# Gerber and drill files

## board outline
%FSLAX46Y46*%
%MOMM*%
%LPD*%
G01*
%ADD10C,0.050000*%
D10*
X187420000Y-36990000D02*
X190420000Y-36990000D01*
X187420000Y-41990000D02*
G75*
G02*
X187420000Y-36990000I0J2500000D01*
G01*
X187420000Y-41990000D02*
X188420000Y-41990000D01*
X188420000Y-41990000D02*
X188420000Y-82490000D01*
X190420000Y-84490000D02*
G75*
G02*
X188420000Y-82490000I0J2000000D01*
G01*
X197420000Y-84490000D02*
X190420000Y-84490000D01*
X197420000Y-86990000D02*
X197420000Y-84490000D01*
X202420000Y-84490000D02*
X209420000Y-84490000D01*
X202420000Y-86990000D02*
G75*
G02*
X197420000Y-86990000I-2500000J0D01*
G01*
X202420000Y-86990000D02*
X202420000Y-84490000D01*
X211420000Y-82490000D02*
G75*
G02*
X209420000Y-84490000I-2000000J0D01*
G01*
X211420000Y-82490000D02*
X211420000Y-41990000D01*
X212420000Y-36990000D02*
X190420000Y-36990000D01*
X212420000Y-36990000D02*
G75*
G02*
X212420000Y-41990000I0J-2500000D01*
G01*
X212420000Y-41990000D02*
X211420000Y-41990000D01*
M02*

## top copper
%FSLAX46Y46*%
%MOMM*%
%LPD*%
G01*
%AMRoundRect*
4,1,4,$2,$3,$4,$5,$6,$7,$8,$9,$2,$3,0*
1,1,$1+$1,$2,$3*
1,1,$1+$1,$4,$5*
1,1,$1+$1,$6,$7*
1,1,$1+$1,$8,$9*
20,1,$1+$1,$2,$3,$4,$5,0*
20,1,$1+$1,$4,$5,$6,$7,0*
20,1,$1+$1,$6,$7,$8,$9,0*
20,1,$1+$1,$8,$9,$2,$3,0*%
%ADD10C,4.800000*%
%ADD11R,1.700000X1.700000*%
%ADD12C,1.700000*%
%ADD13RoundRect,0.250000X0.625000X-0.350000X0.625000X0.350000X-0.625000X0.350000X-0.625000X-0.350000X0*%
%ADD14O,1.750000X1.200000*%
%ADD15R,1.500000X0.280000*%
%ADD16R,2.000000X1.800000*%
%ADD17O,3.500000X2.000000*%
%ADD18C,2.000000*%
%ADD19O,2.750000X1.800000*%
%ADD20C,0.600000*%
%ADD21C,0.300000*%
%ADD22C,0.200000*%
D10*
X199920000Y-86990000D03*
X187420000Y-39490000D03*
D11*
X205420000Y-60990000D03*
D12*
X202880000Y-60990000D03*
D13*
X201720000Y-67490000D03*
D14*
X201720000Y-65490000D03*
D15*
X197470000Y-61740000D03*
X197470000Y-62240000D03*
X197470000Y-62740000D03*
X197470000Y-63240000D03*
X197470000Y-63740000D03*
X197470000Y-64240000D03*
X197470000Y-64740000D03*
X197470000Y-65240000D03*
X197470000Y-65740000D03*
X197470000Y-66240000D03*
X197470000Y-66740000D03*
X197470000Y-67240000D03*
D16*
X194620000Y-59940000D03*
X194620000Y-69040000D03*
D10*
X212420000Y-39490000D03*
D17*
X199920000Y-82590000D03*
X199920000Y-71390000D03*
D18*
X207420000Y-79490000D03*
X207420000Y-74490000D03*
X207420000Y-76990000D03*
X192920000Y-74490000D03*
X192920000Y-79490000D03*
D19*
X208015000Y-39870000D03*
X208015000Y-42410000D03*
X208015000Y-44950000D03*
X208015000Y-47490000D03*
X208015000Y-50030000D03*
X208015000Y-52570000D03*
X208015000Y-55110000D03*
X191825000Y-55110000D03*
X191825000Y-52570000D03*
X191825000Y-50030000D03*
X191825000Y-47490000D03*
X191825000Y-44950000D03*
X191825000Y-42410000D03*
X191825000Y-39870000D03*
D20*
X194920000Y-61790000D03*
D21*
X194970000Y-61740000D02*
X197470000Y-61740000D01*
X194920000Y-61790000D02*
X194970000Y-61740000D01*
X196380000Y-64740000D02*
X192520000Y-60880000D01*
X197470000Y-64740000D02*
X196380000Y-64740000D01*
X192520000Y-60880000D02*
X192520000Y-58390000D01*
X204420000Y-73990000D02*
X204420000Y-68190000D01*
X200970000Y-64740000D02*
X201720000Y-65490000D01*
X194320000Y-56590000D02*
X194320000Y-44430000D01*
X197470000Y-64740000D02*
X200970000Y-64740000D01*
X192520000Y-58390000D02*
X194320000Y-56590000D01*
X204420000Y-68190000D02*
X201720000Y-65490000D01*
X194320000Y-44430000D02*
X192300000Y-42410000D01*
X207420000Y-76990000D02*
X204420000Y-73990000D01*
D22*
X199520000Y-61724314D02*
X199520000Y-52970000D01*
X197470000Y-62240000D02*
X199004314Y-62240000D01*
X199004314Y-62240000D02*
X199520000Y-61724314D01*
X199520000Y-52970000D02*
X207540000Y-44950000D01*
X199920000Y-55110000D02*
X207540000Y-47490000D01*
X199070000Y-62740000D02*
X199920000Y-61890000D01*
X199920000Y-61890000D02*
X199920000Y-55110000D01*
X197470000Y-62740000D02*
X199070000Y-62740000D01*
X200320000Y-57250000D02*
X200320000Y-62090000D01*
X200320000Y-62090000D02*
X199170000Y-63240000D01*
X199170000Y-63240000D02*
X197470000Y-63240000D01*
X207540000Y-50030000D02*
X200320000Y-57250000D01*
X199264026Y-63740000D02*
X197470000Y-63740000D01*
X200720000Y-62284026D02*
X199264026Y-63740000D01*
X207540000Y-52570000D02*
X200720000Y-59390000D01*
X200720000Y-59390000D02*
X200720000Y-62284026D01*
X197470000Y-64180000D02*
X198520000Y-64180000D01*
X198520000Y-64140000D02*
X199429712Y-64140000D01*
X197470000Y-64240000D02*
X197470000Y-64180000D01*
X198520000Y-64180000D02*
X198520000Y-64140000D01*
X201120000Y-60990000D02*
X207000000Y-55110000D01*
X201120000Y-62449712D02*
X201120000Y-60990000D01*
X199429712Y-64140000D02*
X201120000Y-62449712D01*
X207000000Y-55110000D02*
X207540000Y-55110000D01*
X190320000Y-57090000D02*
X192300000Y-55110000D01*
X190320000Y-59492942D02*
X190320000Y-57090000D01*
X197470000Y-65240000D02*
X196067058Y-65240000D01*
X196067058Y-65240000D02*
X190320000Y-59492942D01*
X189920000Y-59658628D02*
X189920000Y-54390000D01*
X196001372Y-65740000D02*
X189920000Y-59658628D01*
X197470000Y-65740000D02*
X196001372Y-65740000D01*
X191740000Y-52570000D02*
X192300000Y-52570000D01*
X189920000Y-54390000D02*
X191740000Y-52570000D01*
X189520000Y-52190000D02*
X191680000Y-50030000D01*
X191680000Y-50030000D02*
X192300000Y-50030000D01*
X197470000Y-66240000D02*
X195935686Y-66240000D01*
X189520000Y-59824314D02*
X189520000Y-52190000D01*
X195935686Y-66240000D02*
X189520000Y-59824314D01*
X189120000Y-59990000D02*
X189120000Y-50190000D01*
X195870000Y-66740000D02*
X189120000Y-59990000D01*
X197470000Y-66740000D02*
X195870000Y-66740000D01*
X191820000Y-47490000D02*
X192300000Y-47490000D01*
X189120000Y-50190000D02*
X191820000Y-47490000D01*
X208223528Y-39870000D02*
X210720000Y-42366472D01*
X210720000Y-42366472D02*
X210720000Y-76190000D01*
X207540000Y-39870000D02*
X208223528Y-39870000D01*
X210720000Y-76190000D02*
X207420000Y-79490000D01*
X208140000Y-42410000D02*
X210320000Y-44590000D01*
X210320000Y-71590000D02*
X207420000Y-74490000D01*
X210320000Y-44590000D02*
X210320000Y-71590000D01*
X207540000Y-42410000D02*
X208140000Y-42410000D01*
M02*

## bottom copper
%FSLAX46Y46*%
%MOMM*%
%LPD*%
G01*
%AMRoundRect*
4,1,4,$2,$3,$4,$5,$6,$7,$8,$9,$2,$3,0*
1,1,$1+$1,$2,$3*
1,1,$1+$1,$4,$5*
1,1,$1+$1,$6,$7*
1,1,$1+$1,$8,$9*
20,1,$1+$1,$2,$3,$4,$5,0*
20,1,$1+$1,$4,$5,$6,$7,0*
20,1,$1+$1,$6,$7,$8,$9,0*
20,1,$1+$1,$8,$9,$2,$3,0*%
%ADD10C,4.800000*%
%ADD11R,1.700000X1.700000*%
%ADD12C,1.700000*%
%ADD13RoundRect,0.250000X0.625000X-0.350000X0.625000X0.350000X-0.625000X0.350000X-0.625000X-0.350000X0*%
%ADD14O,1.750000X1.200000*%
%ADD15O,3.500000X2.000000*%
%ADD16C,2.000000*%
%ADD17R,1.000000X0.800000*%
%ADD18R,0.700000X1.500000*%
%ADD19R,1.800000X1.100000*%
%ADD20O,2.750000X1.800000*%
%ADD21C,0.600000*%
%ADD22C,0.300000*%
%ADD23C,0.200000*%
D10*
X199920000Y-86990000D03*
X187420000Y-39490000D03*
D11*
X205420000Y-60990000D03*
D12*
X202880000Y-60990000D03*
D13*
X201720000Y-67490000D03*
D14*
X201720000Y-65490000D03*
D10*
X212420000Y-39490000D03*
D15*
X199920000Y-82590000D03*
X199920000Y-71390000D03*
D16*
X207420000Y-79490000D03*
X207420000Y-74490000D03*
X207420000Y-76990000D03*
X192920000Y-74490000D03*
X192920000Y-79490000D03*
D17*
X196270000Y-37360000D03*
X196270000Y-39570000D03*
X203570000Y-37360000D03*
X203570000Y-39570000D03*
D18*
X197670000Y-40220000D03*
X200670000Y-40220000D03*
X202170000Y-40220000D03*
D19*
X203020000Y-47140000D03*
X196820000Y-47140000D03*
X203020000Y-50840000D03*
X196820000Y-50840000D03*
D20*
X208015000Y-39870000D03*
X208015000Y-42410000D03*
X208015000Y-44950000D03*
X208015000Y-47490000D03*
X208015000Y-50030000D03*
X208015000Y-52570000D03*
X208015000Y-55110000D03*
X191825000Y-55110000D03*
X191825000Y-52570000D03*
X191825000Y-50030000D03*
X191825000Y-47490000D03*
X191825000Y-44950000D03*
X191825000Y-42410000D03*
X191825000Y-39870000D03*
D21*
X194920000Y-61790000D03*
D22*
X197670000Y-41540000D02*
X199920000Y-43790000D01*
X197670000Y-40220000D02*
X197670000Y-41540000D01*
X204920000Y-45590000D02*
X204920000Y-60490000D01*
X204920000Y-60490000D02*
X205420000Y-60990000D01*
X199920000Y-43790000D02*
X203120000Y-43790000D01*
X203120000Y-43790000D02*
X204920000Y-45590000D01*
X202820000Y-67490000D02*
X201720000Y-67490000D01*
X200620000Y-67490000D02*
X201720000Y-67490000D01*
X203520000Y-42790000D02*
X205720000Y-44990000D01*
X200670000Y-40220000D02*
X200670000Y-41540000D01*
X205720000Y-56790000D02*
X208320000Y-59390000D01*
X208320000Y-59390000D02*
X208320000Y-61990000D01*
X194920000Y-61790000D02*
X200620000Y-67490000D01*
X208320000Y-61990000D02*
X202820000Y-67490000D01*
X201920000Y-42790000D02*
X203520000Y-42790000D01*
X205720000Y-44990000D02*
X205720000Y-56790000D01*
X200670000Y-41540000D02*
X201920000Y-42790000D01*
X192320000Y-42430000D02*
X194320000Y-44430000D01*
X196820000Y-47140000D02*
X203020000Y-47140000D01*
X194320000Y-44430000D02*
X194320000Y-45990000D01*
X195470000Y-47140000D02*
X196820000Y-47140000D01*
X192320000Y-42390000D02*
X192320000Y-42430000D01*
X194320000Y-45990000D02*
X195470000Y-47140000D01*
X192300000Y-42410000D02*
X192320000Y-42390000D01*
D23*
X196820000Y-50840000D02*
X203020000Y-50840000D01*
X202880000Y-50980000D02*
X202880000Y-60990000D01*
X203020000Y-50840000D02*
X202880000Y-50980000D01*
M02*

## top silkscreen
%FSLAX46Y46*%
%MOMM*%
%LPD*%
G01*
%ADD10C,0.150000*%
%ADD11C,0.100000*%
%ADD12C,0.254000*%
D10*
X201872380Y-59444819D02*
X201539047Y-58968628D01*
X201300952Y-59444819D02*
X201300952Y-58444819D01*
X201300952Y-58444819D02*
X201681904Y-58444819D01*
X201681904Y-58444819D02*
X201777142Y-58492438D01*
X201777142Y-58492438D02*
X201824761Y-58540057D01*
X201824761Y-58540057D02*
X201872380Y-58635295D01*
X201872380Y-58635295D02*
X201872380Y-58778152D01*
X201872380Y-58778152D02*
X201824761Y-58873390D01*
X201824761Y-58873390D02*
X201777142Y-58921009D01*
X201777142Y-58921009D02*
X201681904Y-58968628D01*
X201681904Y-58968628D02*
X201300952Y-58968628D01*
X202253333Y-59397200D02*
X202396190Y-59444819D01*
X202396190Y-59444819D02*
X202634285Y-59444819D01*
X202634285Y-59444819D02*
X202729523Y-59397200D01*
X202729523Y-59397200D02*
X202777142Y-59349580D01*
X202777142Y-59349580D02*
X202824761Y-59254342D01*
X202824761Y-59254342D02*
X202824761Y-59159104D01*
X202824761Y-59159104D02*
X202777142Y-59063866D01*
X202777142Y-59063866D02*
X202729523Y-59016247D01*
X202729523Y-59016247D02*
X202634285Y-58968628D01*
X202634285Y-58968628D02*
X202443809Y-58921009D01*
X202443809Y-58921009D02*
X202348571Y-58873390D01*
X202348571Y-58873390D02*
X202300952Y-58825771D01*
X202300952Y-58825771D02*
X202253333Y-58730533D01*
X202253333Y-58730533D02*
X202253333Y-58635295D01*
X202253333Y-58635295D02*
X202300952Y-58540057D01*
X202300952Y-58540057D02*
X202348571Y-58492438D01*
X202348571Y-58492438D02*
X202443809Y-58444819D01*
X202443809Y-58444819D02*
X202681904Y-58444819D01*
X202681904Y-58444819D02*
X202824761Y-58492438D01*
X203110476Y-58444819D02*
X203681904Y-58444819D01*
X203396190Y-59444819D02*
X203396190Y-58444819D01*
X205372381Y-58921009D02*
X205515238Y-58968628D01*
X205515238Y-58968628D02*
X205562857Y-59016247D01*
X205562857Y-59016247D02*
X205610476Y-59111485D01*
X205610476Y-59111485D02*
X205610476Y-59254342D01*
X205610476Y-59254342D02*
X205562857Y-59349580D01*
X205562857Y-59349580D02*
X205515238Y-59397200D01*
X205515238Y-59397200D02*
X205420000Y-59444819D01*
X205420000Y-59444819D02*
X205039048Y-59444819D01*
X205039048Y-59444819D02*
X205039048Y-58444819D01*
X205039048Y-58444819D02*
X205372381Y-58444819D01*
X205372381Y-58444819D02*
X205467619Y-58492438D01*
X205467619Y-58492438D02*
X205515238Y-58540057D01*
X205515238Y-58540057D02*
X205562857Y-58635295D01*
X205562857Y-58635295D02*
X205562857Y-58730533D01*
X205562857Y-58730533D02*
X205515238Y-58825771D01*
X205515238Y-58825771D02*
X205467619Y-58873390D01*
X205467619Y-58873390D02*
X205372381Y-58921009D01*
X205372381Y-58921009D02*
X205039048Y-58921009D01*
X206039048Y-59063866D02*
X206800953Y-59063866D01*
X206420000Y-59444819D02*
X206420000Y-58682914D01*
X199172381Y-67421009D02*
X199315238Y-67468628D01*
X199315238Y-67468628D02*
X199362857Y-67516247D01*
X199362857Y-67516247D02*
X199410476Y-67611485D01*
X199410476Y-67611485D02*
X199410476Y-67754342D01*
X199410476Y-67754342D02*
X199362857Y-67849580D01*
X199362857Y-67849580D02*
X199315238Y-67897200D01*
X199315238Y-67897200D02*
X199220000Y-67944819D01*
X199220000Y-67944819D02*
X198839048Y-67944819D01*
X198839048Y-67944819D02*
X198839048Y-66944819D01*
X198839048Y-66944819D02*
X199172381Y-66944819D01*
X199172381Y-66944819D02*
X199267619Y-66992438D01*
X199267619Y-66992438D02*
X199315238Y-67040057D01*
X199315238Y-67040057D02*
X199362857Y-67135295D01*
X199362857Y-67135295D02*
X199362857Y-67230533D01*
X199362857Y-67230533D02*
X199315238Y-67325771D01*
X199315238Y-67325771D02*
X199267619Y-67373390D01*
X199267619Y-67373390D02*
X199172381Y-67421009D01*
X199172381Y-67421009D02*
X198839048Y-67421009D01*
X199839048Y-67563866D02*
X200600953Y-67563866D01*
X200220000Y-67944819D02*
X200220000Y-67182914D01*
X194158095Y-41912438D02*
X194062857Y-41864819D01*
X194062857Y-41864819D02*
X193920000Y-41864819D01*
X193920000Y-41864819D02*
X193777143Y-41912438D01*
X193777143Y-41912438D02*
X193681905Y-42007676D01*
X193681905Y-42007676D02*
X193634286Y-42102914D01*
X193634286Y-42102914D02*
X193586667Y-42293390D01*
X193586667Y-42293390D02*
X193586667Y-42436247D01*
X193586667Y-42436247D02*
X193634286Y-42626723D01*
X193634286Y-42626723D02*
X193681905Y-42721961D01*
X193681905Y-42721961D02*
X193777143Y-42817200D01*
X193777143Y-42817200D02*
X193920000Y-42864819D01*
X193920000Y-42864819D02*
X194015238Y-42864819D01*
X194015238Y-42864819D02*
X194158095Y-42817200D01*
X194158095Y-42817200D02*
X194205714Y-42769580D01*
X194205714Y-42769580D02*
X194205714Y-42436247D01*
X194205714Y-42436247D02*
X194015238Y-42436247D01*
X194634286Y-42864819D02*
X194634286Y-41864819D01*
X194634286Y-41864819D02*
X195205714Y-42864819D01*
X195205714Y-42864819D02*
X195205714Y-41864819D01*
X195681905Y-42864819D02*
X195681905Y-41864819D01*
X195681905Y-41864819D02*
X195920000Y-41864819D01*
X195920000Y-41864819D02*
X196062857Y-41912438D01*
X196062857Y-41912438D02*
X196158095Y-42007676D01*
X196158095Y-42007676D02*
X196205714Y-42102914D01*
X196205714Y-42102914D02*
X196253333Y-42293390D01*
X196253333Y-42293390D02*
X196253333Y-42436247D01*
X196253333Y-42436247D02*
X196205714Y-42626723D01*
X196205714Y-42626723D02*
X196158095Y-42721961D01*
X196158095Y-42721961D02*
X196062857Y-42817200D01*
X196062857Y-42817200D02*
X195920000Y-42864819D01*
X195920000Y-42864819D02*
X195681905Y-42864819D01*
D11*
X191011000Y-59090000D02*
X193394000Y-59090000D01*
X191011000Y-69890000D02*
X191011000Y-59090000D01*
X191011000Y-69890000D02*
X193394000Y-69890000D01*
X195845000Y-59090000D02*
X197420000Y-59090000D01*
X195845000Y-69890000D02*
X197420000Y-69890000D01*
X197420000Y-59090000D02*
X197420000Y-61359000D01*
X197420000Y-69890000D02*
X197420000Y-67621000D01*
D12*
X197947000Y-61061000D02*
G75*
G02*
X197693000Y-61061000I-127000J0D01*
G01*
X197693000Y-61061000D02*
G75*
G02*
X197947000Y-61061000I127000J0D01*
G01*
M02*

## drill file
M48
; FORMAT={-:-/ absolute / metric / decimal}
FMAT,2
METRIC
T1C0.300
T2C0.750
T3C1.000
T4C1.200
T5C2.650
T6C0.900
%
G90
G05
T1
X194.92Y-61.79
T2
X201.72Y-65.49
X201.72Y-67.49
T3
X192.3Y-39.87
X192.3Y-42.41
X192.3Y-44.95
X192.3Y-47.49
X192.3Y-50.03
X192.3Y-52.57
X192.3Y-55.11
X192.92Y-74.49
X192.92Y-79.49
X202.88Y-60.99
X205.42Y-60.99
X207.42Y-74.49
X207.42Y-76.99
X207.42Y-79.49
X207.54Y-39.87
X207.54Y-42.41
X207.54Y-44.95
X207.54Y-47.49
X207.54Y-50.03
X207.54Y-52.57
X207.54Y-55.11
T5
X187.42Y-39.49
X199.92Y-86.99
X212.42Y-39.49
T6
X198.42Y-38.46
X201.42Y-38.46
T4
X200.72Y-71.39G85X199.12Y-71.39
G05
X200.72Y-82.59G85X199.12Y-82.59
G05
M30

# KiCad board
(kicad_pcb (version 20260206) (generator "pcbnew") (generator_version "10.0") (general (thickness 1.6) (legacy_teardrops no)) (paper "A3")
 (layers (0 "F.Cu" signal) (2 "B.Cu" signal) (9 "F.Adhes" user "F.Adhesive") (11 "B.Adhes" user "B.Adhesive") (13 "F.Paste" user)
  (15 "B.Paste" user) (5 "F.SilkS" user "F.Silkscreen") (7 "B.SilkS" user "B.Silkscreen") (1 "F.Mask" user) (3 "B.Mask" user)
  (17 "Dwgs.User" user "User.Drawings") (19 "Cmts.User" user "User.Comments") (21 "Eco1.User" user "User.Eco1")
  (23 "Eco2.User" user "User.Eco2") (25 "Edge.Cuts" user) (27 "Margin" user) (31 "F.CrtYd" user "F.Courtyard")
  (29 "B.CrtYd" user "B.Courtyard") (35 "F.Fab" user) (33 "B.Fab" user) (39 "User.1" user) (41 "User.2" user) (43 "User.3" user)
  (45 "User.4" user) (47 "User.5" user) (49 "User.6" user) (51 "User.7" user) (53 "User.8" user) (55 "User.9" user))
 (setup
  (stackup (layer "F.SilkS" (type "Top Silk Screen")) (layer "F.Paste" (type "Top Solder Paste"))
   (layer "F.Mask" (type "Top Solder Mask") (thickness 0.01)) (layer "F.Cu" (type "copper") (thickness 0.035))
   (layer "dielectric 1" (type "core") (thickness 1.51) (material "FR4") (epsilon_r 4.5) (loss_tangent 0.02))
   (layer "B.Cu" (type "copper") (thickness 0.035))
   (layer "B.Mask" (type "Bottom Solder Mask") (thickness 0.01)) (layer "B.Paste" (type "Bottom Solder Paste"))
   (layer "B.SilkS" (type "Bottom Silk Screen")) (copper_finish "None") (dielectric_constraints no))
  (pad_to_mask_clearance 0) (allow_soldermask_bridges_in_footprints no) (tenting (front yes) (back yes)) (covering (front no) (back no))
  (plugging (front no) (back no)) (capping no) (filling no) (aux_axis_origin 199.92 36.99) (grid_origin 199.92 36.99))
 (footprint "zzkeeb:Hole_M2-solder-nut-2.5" (layer "F.Cu") (at 199.92 86.99)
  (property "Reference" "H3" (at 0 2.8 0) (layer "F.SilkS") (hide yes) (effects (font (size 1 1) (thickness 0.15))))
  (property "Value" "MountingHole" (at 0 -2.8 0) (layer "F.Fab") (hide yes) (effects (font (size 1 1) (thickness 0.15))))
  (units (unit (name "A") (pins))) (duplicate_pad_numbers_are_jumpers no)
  (pad "" thru_hole circle (at 0 0) (size 4.8 4.8) (drill 2.65) (layers "*.Cu" "F.Mask") (remove_unused_layers no)))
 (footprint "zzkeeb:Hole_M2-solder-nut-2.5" (layer "F.Cu") (at 187.42 39.49)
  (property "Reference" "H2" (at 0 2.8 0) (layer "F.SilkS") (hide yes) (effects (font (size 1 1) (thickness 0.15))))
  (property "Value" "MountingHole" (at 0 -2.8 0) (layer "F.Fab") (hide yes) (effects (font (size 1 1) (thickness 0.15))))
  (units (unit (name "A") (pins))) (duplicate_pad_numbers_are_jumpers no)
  (pad "" thru_hole circle (at 0 0) (size 4.8 4.8) (drill 2.65) (layers "*.Cu" "F.Mask") (remove_unused_layers no)))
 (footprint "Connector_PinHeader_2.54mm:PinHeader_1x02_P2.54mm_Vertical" (layer "F.Cu") (at 205.42 60.99 -90)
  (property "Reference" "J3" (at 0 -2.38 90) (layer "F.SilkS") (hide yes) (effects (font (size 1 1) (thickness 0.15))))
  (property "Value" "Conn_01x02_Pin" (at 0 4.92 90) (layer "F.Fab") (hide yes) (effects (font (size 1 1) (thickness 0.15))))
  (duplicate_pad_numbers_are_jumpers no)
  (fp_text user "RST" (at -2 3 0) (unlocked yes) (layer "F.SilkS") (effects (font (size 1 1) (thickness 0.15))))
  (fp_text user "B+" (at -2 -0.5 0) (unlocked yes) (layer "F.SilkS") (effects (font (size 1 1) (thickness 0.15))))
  (pad "1" thru_hole rect (at 0 0 270) (size 1.7 1.7) (drill 1) (layers "*.Cu" "*.Mask") (remove_unused_layers no) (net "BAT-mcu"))
  (pad "2" thru_hole circle (at 0 2.54 270) (size 1.7 1.7) (drill 1) (layers "*.Cu" "*.Mask") (remove_unused_layers no) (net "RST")))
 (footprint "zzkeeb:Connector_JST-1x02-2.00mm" (layer "F.Cu") (at 201.72 67.49 90)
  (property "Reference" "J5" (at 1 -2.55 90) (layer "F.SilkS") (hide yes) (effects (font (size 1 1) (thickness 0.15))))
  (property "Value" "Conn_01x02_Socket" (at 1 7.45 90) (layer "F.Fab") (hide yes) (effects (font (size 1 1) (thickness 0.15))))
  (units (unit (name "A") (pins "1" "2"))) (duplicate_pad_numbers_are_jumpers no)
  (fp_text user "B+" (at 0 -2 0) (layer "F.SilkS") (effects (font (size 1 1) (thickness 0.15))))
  (pad "1" thru_hole roundrect (at 0 0 90) (size 1.2 1.75) (drill 0.75) (layers "*.Cu" "*.Mask") (remove_unused_layers no)
   (roundrect_rratio 0.208333) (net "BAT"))
  (pad "2" thru_hole oval (at 2 0 90) (size 1.2 1.75) (drill 0.75) (layers "*.Cu" "*.Mask") (remove_unused_layers no) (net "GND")))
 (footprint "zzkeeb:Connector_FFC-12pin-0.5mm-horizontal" (layer "F.Cu") (at 195.92 64.49 -90)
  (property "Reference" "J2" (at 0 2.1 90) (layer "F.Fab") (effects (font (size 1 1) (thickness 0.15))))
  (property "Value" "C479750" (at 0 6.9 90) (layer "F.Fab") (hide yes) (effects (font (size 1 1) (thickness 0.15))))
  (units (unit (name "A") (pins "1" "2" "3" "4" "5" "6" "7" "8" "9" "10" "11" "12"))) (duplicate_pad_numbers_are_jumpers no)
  (fp_line (start -5.4 4.909) (end -5.4 2.526) (stroke (width 0.1) (type solid)) (layer "F.SilkS"))
  (fp_line (start 5.4 4.909) (end -5.4 4.909) (stroke (width 0.1) (type solid)) (layer "F.SilkS"))
  (fp_line (start 5.4 4.909) (end 5.4 2.526) (stroke (width 0.1) (type solid)) (layer "F.SilkS"))
  (fp_line (start -5.4 0.075) (end -5.4 -1.5) (stroke (width 0.1) (type solid)) (layer "F.SilkS"))
  (fp_line (start 5.4 0.075) (end 5.4 -1.5) (stroke (width 0.1) (type solid)) (layer "F.SilkS"))
  (fp_line (start -5.4 -1.5) (end -3.131 -1.5) (stroke (width 0.1) (type solid)) (layer "F.SilkS"))
  (fp_line (start 5.4 -1.5) (end 3.131 -1.5) (stroke (width 0.1) (type solid)) (layer "F.SilkS"))
  (fp_circle (center -3.429 -1.9) (end -3.302 -1.9) (stroke (width 0.254) (type solid)) (fill no) (layer "F.SilkS"))
  (pad "1" smd rect (at -2.75 -1.55 270) (size 0.28 1.5) (layers "F.Cu" "F.Mask" "F.Paste") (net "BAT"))
  (pad "2" smd rect (at -2.25 -1.55 270) (size 0.28 1.5) (layers "F.Cu" "F.Mask" "F.Paste") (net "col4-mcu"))
  (pad "3" smd rect (at -1.75 -1.55 270) (size 0.28 1.5) (layers "F.Cu" "F.Mask" "F.Paste") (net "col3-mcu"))
  (pad "4" smd rect (at -1.25 -1.55 270) (size 0.28 1.5) (layers "F.Cu" "F.Mask" "F.Paste") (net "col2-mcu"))
  (pad "5" smd rect (at -0.75 -1.55 270) (size 0.28 1.5) (layers "F.Cu" "F.Mask" "F.Paste") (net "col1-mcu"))
  (pad "6" smd rect (at -0.25 -1.55 270) (size 0.28 1.5) (layers "F.Cu" "F.Mask" "F.Paste") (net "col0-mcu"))
  (pad "7" smd rect (at 0.25 -1.55 270) (size 0.28 1.5) (layers "F.Cu" "F.Mask" "F.Paste") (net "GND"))
  (pad "8" smd rect (at 0.75 -1.55 270) (size 0.28 1.5) (layers "F.Cu" "F.Mask" "F.Paste") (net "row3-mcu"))
  (pad "9" smd rect (at 1.25 -1.55 270) (size 0.28 1.5) (layers "F.Cu" "F.Mask" "F.Paste") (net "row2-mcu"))
  (pad "10" smd rect (at 1.75 -1.55 270) (size 0.28 1.5) (layers "F.Cu" "F.Mask" "F.Paste") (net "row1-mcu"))
  (pad "11" smd rect (at 2.25 -1.55 270) (size 0.28 1.5) (layers "F.Cu" "F.Mask" "F.Paste") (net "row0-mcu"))
  (pad "12" smd rect (at 2.75 -1.55 270) (size 0.28 1.5) (layers "F.Cu" "F.Mask" "F.Paste") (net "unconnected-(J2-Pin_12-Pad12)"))
  (pad "MP" smd rect (at -4.55 1.3 270) (size 1.8 2) (layers "F.Cu" "F.Mask" "F.Paste"))
  (pad "MP" smd rect (at 4.55 1.3 270) (size 1.8 2) (layers "F.Cu" "F.Mask" "F.Paste")))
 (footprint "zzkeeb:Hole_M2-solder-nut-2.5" (layer "F.Cu") (at 212.42 39.49)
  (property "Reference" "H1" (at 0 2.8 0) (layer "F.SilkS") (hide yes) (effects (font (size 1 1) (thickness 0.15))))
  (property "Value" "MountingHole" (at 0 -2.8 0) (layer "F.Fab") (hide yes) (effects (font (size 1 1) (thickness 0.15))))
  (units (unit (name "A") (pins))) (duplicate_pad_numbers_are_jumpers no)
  (pad "" thru_hole circle (at 0 0) (size 4.8 4.8) (drill 2.65) (layers "*.Cu" "F.Mask") (remove_unused_layers no)))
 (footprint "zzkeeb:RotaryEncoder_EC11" (layer "F.Cu") (at 199.92 76.99 180)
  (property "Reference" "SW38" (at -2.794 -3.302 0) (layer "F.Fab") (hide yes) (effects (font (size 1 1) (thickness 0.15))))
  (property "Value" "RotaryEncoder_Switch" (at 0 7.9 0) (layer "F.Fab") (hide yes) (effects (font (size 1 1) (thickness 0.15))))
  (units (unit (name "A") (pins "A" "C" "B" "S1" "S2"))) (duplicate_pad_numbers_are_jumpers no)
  (pad "" thru_hole oval (at 0 -5.6 180) (size 3.5 2) (drill oval 2.8 1.2) (layers "*.Cu" "*.Mask") (remove_unused_layers no))
  (pad "" thru_hole oval (at 0 5.6 180) (size 3.5 2) (drill oval 2.8 1.2) (layers "*.Cu" "*.Mask") (remove_unused_layers no))
  (pad "A" thru_hole circle (at -7.5 -2.5 180) (size 2 2) (drill 1) (layers "*.Cu" "B.Mask") (remove_unused_layers no) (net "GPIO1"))
  (pad "B" thru_hole circle (at -7.5 2.5 180) (size 2 2) (drill 1) (layers "*.Cu" "B.Mask") (remove_unused_layers no) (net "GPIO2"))
  (pad "C" thru_hole circle (at -7.5 0 180) (size 2 2) (drill 1) (layers "*.Cu" "B.Mask") (remove_unused_layers no) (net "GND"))
  (pad "S1" thru_hole circle (at 7 2.5 180) (size 2 2) (drill 1) (layers "*.Cu" "B.Mask") (remove_unused_layers no)
   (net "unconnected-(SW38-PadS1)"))
  (pad "S2" thru_hole circle (at 7 -2.5 180) (size 2 2) (drill 1) (layers "*.Cu" "B.Mask") (remove_unused_layers no)
   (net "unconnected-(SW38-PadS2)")))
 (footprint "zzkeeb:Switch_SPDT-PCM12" (layer "B.Cu") (at 199.92 38.79)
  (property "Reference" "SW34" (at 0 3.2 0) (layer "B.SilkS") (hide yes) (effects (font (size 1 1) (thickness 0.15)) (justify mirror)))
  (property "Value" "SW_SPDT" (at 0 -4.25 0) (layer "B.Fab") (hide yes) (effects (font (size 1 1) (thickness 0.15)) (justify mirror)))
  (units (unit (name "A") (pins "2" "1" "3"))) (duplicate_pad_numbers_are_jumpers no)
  (pad "" smd rect (at -3.65 -1.43) (size 1 0.8) (layers "B.Cu" "B.Mask" "B.Paste"))
  (pad "" smd rect (at -3.65 0.78) (size 1 0.8) (layers "B.Cu" "B.Mask" "B.Paste"))
  (pad "" np_thru_hole circle (at -1.5 -0.33) (size 0.9 0.9) (drill 0.9) (layers "*.Cu" "*.Mask"))
  (pad "" np_thru_hole circle (at 1.5 -0.33) (size 0.9 0.9) (drill 0.9) (layers "*.Cu" "*.Mask"))
  (pad "" smd rect (at 3.65 -1.43) (size 1 0.8) (layers "B.Cu" "B.Mask" "B.Paste"))
  (pad "" smd rect (at 3.65 0.78) (size 1 0.8) (layers "B.Cu" "B.Mask" "B.Paste"))
  (pad "1" smd rect (at -2.25 1.43) (size 0.7 1.5) (layers "B.Cu" "B.Mask" "B.Paste") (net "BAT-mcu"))
  (pad "2" smd rect (at 0.75 1.43) (size 0.7 1.5) (layers "B.Cu" "B.Mask" "B.Paste") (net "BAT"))
  (pad "3" smd rect (at 2.25 1.43) (size 0.7 1.5) (layers "B.Cu" "B.Mask" "B.Paste") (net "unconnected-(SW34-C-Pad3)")))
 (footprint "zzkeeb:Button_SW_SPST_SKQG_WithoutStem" (layer "B.Cu") (at 199.92 48.99 180)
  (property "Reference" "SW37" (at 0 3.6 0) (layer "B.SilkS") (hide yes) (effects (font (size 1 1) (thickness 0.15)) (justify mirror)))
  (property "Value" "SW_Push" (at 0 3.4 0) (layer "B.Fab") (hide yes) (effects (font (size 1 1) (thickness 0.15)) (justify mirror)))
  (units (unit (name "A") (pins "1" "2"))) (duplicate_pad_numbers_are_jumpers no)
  (pad "1" smd rect (at -3.1 1.85 180) (size 1.8 1.1) (layers "B.Cu" "B.Mask" "B.Paste") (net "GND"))
  (pad "1" smd rect (at 3.1 1.85 180) (size 1.8 1.1) (layers "B.Cu" "B.Mask" "B.Paste") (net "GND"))
  (pad "2" smd rect (at -3.1 -1.85 180) (size 1.8 1.1) (layers "B.Cu" "B.Mask" "B.Paste") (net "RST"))
  (pad "2" smd rect (at 3.1 -1.85 180) (size 1.8 1.1) (layers "B.Cu" "B.Mask" "B.Paste") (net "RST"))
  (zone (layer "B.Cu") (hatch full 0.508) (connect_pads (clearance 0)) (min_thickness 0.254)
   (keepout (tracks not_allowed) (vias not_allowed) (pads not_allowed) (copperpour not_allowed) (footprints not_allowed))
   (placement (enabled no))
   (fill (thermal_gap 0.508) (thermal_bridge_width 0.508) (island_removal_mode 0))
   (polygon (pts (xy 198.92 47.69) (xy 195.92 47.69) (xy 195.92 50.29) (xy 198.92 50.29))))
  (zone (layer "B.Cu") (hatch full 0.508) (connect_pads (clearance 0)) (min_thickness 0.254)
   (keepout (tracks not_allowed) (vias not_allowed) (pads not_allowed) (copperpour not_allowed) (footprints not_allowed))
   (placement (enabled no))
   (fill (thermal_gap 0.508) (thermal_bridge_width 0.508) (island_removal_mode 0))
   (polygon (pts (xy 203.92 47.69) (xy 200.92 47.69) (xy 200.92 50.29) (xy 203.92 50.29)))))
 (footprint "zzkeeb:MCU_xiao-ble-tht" (layer "B.Cu") (at 199.92 47.49 180)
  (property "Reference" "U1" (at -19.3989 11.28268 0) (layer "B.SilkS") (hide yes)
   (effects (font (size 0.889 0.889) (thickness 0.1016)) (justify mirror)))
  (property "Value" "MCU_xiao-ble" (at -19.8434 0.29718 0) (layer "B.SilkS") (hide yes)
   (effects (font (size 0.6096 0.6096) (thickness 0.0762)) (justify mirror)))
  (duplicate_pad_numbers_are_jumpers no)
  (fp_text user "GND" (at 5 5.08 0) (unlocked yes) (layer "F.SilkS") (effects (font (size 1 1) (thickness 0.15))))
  (pad "1" thru_hole oval (at -7.62 7.62 180) (size 2.75 1.8) (drill 1 (offset -0.475 0)) (layers "*.Cu" "*.Mask") (remove_unused_layers no)
   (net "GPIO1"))
  (pad "2" thru_hole oval (at -7.62 5.08 180) (size 2.75 1.8) (drill 1 (offset -0.475 0)) (layers "*.Cu" "*.Mask") (remove_unused_layers no)
   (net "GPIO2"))
  (pad "3" thru_hole oval (at -7.62 2.54 180) (size 2.75 1.8) (drill 1 (offset -0.475 0)) (layers "*.Cu" "*.Mask") (remove_unused_layers no)
   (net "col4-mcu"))
  (pad "4" thru_hole oval (at -7.62 0 180) (size 2.75 1.8) (drill 1 (offset -0.475 0)) (layers "*.Cu" "*.Mask") (remove_unused_layers no)
   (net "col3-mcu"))
  (pad "5" thru_hole oval (at -7.62 -2.54 180) (size 2.75 1.8) (drill 1 (offset -0.475 0)) (layers "*.Cu" "*.Mask")
   (remove_unused_layers no) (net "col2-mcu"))
  (pad "6" thru_hole oval (at -7.62 -5.08 180) (size 2.75 1.8) (drill 1 (offset -0.475 0)) (layers "*.Cu" "*.Mask")
   (remove_unused_layers no) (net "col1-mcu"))
  (pad "7" thru_hole oval (at -7.62 -7.62 180) (size 2.75 1.8) (drill 1 (offset -0.475 0)) (layers "*.Cu" "*.Mask")
   (remove_unused_layers no) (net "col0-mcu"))
  (pad "8" thru_hole oval (at 7.62 -7.62) (size 2.75 1.8) (drill 1 (offset -0.475 0)) (layers "*.Cu" "*.Mask") (remove_unused_layers no)
   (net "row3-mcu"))
  (pad "9" thru_hole oval (at 7.62 -5.08) (size 2.75 1.8) (drill 1 (offset -0.475 0)) (layers "*.Cu" "*.Mask") (remove_unused_layers no)
   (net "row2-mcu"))
  (pad "10" thru_hole oval (at 7.62 -2.54) (size 2.75 1.8) (drill 1 (offset -0.475 0)) (layers "*.Cu" "*.Mask") (remove_unused_layers no)
   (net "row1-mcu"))
  (pad "11" thru_hole oval (at 7.62 0) (size 2.75 1.8) (drill 1 (offset -0.475 0)) (layers "*.Cu" "*.Mask") (remove_unused_layers no)
   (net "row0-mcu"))
  (pad "12" thru_hole oval (at 7.62 2.54) (size 2.75 1.8) (drill 1 (offset -0.475 0)) (layers "*.Cu" "*.Mask") (remove_unused_layers no)
   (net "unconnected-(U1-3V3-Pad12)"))
  (pad "13" thru_hole oval (at 7.62 5.08) (size 2.75 1.8) (drill 1 (offset -0.475 0)) (layers "*.Cu" "*.Mask") (remove_unused_layers no)
   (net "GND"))
  (pad "14" thru_hole oval (at 7.62 7.62) (size 2.75 1.8) (drill 1 (offset -0.475 0)) (layers "*.Cu" "*.Mask") (remove_unused_layers no)
   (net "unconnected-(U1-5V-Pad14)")))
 (gr_line (start 187.42 36.99) (end 190.42 36.99) (stroke (width 0.05) (type default)) (layer "Edge.Cuts"))
 (gr_arc (start 187.42 41.99) (mid 184.92 39.49) (end 187.42 36.99) (stroke (width 0.05) (type default)) (layer "Edge.Cuts"))
 (gr_line (start 187.42 41.99) (end 188.42 41.99) (stroke (width 0.05) (type default)) (layer "Edge.Cuts"))
 (gr_line (start 188.42 41.99) (end 188.42 82.49) (stroke (width 0.05) (type default)) (layer "Edge.Cuts"))
 (gr_arc (start 190.42 84.49) (mid 189.005786 83.904214) (end 188.42 82.49) (stroke (width 0.05) (type default)) (layer "Edge.Cuts"))
 (gr_line (start 197.42 84.49) (end 190.42 84.49) (stroke (width 0.05) (type default)) (layer "Edge.Cuts"))
 (gr_line (start 197.42 86.99) (end 197.42 84.49) (stroke (width 0.05) (type default)) (layer "Edge.Cuts"))
 (gr_line (start 202.42 84.49) (end 209.42 84.49) (stroke (width 0.05) (type default)) (layer "Edge.Cuts"))
 (gr_arc (start 202.42 86.99) (mid 199.92 89.49) (end 197.42 86.99) (stroke (width 0.05) (type default)) (layer "Edge.Cuts"))
 (gr_line (start 202.42 86.99) (end 202.42 84.49) (stroke (width 0.05) (type default)) (layer "Edge.Cuts"))
 (gr_arc (start 211.42 82.49) (mid 210.834214 83.904214) (end 209.42 84.49) (stroke (width 0.05) (type default)) (layer "Edge.Cuts"))
 (gr_line (start 211.42 82.49) (end 211.42 41.99) (stroke (width 0.05) (type default)) (layer "Edge.Cuts"))
 (gr_line (start 212.42 36.99) (end 190.42 36.99) (stroke (width 0.05) (type default)) (layer "Edge.Cuts"))
 (gr_arc (start 212.42 36.99) (mid 214.92 39.49) (end 212.42 41.99) (stroke (width 0.05) (type default)) (layer "Edge.Cuts"))
 (gr_line (start 212.42 41.99) (end 211.42 41.99) (stroke (width 0.05) (type default)) (layer "Edge.Cuts"))
 (segment (start 197.67 41.54) (end 199.92 43.79) (width 0.3) (layer "B.Cu") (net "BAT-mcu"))
 (segment (start 197.67 40.22) (end 197.67 41.54) (width 0.3) (layer "B.Cu") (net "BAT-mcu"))
 (segment (start 204.92 45.59) (end 204.92 60.49) (width 0.3) (layer "B.Cu") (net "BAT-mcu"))
 (segment (start 204.92 60.49) (end 205.42 60.99) (width 0.3) (layer "B.Cu") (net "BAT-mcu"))
 (segment (start 199.92 43.79) (end 203.12 43.79) (width 0.3) (layer "B.Cu") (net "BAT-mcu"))
 (segment (start 203.12 43.79) (end 204.92 45.59) (width 0.3) (layer "B.Cu") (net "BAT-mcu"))
 (segment (start 194.97 61.74) (end 197.47 61.74) (width 0.3) (layer "F.Cu") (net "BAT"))
 (segment (start 194.92 61.79) (end 194.97 61.74) (width 0.3) (layer "F.Cu") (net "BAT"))
 (via (at 194.92 61.79) (size 0.6) (drill 0.3) (layers "F.Cu" "B.Cu") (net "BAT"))
 (segment (start 202.82 67.49) (end 201.72 67.49) (width 0.3) (layer "B.Cu") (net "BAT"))
 (segment (start 200.62 67.49) (end 201.72 67.49) (width 0.3) (layer "B.Cu") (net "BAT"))
 (segment (start 203.52 42.79) (end 205.72 44.99) (width 0.3) (layer "B.Cu") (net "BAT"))
 (segment (start 200.67 40.22) (end 200.67 41.54) (width 0.3) (layer "B.Cu") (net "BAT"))
 (segment (start 205.72 56.79) (end 208.32 59.39) (width 0.3) (layer "B.Cu") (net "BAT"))
 (segment (start 208.32 59.39) (end 208.32 61.99) (width 0.3) (layer "B.Cu") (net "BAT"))
 (segment (start 194.92 61.79) (end 200.62 67.49) (width 0.3) (layer "B.Cu") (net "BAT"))
 (segment (start 208.32 61.99) (end 202.82 67.49) (width 0.3) (layer "B.Cu") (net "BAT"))
 (segment (start 201.92 42.79) (end 203.52 42.79) (width 0.3) (layer "B.Cu") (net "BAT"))
 (segment (start 205.72 44.99) (end 205.72 56.79) (width 0.3) (layer "B.Cu") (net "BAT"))
 (segment (start 200.67 41.54) (end 201.92 42.79) (width 0.3) (layer "B.Cu") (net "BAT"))
 (segment (start 196.38 64.74) (end 192.52 60.88) (width 0.3) (layer "F.Cu") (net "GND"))
 (segment (start 197.47 64.74) (end 196.38 64.74) (width 0.3) (layer "F.Cu") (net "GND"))
 (segment (start 192.52 60.88) (end 192.52 58.39) (width 0.3) (layer "F.Cu") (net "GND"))
 (segment (start 204.42 73.99) (end 204.42 68.19) (width 0.3) (layer "F.Cu") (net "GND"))
 (segment (start 200.97 64.74) (end 201.72 65.49) (width 0.3) (layer "F.Cu") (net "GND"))
 (segment (start 194.32 56.59) (end 194.32 44.43) (width 0.3) (layer "F.Cu") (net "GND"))
 (segment (start 197.47 64.74) (end 200.97 64.74) (width 0.3) (layer "F.Cu") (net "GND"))
 (segment (start 192.52 58.39) (end 194.32 56.59) (width 0.3) (layer "F.Cu") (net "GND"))
 (segment (start 204.42 68.19) (end 201.72 65.49) (width 0.3) (layer "F.Cu") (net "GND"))
 (segment (start 194.32 44.43) (end 192.3 42.41) (width 0.3) (layer "F.Cu") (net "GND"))
 (segment (start 207.42 76.99) (end 204.42 73.99) (width 0.3) (layer "F.Cu") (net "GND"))
 (segment (start 192.32 42.43) (end 194.32 44.43) (width 0.3) (layer "B.Cu") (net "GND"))
 (segment (start 196.82 47.14) (end 203.02 47.14) (width 0.3) (layer "B.Cu") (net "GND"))
 (segment (start 194.32 44.43) (end 194.32 45.99) (width 0.3) (layer "B.Cu") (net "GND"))
 (segment (start 195.47 47.14) (end 196.82 47.14) (width 0.3) (layer "B.Cu") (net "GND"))
 (segment (start 192.32 42.39) (end 192.32 42.43) (width 0.3) (layer "B.Cu") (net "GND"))
 (segment (start 194.32 45.99) (end 195.47 47.14) (width 0.3) (layer "B.Cu") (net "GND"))
 (segment (start 192.3 42.41) (end 192.32 42.39) (width 0.3) (layer "B.Cu") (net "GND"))
 (segment (start 199.52 61.724314) (end 199.52 52.97) (width 0.2) (layer "F.Cu") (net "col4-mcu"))
 (segment (start 197.47 62.24) (end 199.004314 62.24) (width 0.2) (layer "F.Cu") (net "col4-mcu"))
 (segment (start 199.004314 62.24) (end 199.52 61.724314) (width 0.2) (layer "F.Cu") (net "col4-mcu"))
 (segment (start 199.52 52.97) (end 207.54 44.95) (width 0.2) (layer "F.Cu") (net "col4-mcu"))
 (segment (start 199.92 55.11) (end 207.54 47.49) (width 0.2) (layer "F.Cu") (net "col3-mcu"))
 (segment (start 199.07 62.74) (end 199.92 61.89) (width 0.2) (layer "F.Cu") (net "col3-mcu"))
 (segment (start 199.92 61.89) (end 199.92 55.11) (width 0.2) (layer "F.Cu") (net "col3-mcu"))
 (segment (start 197.47 62.74) (end 199.07 62.74) (width 0.2) (layer "F.Cu") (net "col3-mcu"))
 (segment (start 200.32 57.25) (end 200.32 62.09) (width 0.2) (layer "F.Cu") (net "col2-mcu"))
 (segment (start 200.32 62.09) (end 199.17 63.24) (width 0.2) (layer "F.Cu") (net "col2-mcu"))
 (segment (start 199.17 63.24) (end 197.47 63.24) (width 0.2) (layer "F.Cu") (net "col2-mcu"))
 (segment (start 207.54 50.03) (end 200.32 57.25) (width 0.2) (layer "F.Cu") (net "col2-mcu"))
 (segment (start 199.264026 63.74) (end 197.47 63.74) (width 0.2) (layer "F.Cu") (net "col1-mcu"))
 (segment (start 200.72 62.284026) (end 199.264026 63.74) (width 0.2) (layer "F.Cu") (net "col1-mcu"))
 (segment (start 207.54 52.57) (end 200.72 59.39) (width 0.2) (layer "F.Cu") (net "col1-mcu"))
 (segment (start 200.72 59.39) (end 200.72 62.284026) (width 0.2) (layer "F.Cu") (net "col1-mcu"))
 (segment (start 197.47 64.18) (end 198.52 64.18) (width 0.2) (layer "F.Cu") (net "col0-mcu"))
 (segment (start 198.52 64.14) (end 199.429712 64.14) (width 0.2) (layer "F.Cu") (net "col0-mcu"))
 (segment (start 197.47 64.24) (end 197.47 64.18) (width 0.2) (layer "F.Cu") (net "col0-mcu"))
 (segment (start 198.52 64.18) (end 198.52 64.14) (width 0.2) (layer "F.Cu") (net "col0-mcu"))
 (segment (start 201.12 60.99) (end 207 55.11) (width 0.2) (layer "F.Cu") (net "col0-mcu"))
 (segment (start 201.12 62.449712) (end 201.12 60.99) (width 0.2) (layer "F.Cu") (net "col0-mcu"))
 (segment (start 199.429712 64.14) (end 201.12 62.449712) (width 0.2) (layer "F.Cu") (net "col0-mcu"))
 (segment (start 207 55.11) (end 207.54 55.11) (width 0.2) (layer "F.Cu") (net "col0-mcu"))
 (segment (start 190.32 57.09) (end 192.3 55.11) (width 0.2) (layer "F.Cu") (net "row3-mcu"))
 (segment (start 190.32 59.492942) (end 190.32 57.09) (width 0.2) (layer "F.Cu") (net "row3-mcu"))
 (segment (start 197.47 65.24) (end 196.067058 65.24) (width 0.2) (layer "F.Cu") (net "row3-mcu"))
 (segment (start 196.067058 65.24) (end 190.32 59.492942) (width 0.2) (layer "F.Cu") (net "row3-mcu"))
 (segment (start 189.92 59.658628) (end 189.92 54.39) (width 0.2) (layer "F.Cu") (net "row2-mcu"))
 (segment (start 196.001372 65.74) (end 189.92 59.658628) (width 0.2) (layer "F.Cu") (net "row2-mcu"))
 (segment (start 197.47 65.74) (end 196.001372 65.74) (width 0.2) (layer "F.Cu") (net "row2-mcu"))
 (segment (start 191.74 52.57) (end 192.3 52.57) (width 0.2) (layer "F.Cu") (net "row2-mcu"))
 (segment (start 189.92 54.39) (end 191.74 52.57) (width 0.2) (layer "F.Cu") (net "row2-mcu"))
 (segment (start 189.52 52.19) (end 191.68 50.03) (width 0.2) (layer "F.Cu") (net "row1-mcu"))
 (segment (start 191.68 50.03) (end 192.3 50.03) (width 0.2) (layer "F.Cu") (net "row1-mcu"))
 (segment (start 197.47 66.24) (end 195.935686 66.24) (width 0.2) (layer "F.Cu") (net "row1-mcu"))
 (segment (start 189.52 59.824314) (end 189.52 52.19) (width 0.2) (layer "F.Cu") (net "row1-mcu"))
 (segment (start 195.935686 66.24) (end 189.52 59.824314) (width 0.2) (layer "F.Cu") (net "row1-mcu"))
 (segment (start 189.12 59.99) (end 189.12 50.19) (width 0.2) (layer "F.Cu") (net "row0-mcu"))
 (segment (start 195.87 66.74) (end 189.12 59.99) (width 0.2) (layer "F.Cu") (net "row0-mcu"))
 (segment (start 197.47 66.74) (end 195.87 66.74) (width 0.2) (layer "F.Cu") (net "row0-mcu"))
 (segment (start 191.82 47.49) (end 192.3 47.49) (width 0.2) (layer "F.Cu") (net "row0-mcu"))
 (segment (start 189.12 50.19) (end 191.82 47.49) (width 0.2) (layer "F.Cu") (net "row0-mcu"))
 (segment (start 208.223528 39.87) (end 210.72 42.366472) (width 0.2) (layer "F.Cu") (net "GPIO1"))
 (segment (start 210.72 42.366472) (end 210.72 76.19) (width 0.2) (layer "F.Cu") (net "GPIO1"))
 (segment (start 207.54 39.87) (end 208.223528 39.87) (width 0.2) (layer "F.Cu") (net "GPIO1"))
 (segment (start 210.72 76.19) (end 207.42 79.49) (width 0.2) (layer "F.Cu") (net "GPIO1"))
 (segment (start 208.14 42.41) (end 210.32 44.59) (width 0.2) (layer "F.Cu") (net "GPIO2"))
 (segment (start 210.32 71.59) (end 207.42 74.49) (width 0.2) (layer "F.Cu") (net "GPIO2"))
 (segment (start 210.32 44.59) (end 210.32 71.59) (width 0.2) (layer "F.Cu") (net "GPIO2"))
 (segment (start 207.54 42.41) (end 208.14 42.41) (width 0.2) (layer "F.Cu") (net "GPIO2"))
 (segment (start 196.82 50.84) (end 203.02 50.84) (width 0.2) (layer "B.Cu") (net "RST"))
 (segment (start 202.88 50.98) (end 202.88 60.99) (width 0.2) (layer "B.Cu") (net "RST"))
 (segment (start 203.02 50.84) (end 202.88 50.98) (width 0.2) (layer "B.Cu") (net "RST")))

